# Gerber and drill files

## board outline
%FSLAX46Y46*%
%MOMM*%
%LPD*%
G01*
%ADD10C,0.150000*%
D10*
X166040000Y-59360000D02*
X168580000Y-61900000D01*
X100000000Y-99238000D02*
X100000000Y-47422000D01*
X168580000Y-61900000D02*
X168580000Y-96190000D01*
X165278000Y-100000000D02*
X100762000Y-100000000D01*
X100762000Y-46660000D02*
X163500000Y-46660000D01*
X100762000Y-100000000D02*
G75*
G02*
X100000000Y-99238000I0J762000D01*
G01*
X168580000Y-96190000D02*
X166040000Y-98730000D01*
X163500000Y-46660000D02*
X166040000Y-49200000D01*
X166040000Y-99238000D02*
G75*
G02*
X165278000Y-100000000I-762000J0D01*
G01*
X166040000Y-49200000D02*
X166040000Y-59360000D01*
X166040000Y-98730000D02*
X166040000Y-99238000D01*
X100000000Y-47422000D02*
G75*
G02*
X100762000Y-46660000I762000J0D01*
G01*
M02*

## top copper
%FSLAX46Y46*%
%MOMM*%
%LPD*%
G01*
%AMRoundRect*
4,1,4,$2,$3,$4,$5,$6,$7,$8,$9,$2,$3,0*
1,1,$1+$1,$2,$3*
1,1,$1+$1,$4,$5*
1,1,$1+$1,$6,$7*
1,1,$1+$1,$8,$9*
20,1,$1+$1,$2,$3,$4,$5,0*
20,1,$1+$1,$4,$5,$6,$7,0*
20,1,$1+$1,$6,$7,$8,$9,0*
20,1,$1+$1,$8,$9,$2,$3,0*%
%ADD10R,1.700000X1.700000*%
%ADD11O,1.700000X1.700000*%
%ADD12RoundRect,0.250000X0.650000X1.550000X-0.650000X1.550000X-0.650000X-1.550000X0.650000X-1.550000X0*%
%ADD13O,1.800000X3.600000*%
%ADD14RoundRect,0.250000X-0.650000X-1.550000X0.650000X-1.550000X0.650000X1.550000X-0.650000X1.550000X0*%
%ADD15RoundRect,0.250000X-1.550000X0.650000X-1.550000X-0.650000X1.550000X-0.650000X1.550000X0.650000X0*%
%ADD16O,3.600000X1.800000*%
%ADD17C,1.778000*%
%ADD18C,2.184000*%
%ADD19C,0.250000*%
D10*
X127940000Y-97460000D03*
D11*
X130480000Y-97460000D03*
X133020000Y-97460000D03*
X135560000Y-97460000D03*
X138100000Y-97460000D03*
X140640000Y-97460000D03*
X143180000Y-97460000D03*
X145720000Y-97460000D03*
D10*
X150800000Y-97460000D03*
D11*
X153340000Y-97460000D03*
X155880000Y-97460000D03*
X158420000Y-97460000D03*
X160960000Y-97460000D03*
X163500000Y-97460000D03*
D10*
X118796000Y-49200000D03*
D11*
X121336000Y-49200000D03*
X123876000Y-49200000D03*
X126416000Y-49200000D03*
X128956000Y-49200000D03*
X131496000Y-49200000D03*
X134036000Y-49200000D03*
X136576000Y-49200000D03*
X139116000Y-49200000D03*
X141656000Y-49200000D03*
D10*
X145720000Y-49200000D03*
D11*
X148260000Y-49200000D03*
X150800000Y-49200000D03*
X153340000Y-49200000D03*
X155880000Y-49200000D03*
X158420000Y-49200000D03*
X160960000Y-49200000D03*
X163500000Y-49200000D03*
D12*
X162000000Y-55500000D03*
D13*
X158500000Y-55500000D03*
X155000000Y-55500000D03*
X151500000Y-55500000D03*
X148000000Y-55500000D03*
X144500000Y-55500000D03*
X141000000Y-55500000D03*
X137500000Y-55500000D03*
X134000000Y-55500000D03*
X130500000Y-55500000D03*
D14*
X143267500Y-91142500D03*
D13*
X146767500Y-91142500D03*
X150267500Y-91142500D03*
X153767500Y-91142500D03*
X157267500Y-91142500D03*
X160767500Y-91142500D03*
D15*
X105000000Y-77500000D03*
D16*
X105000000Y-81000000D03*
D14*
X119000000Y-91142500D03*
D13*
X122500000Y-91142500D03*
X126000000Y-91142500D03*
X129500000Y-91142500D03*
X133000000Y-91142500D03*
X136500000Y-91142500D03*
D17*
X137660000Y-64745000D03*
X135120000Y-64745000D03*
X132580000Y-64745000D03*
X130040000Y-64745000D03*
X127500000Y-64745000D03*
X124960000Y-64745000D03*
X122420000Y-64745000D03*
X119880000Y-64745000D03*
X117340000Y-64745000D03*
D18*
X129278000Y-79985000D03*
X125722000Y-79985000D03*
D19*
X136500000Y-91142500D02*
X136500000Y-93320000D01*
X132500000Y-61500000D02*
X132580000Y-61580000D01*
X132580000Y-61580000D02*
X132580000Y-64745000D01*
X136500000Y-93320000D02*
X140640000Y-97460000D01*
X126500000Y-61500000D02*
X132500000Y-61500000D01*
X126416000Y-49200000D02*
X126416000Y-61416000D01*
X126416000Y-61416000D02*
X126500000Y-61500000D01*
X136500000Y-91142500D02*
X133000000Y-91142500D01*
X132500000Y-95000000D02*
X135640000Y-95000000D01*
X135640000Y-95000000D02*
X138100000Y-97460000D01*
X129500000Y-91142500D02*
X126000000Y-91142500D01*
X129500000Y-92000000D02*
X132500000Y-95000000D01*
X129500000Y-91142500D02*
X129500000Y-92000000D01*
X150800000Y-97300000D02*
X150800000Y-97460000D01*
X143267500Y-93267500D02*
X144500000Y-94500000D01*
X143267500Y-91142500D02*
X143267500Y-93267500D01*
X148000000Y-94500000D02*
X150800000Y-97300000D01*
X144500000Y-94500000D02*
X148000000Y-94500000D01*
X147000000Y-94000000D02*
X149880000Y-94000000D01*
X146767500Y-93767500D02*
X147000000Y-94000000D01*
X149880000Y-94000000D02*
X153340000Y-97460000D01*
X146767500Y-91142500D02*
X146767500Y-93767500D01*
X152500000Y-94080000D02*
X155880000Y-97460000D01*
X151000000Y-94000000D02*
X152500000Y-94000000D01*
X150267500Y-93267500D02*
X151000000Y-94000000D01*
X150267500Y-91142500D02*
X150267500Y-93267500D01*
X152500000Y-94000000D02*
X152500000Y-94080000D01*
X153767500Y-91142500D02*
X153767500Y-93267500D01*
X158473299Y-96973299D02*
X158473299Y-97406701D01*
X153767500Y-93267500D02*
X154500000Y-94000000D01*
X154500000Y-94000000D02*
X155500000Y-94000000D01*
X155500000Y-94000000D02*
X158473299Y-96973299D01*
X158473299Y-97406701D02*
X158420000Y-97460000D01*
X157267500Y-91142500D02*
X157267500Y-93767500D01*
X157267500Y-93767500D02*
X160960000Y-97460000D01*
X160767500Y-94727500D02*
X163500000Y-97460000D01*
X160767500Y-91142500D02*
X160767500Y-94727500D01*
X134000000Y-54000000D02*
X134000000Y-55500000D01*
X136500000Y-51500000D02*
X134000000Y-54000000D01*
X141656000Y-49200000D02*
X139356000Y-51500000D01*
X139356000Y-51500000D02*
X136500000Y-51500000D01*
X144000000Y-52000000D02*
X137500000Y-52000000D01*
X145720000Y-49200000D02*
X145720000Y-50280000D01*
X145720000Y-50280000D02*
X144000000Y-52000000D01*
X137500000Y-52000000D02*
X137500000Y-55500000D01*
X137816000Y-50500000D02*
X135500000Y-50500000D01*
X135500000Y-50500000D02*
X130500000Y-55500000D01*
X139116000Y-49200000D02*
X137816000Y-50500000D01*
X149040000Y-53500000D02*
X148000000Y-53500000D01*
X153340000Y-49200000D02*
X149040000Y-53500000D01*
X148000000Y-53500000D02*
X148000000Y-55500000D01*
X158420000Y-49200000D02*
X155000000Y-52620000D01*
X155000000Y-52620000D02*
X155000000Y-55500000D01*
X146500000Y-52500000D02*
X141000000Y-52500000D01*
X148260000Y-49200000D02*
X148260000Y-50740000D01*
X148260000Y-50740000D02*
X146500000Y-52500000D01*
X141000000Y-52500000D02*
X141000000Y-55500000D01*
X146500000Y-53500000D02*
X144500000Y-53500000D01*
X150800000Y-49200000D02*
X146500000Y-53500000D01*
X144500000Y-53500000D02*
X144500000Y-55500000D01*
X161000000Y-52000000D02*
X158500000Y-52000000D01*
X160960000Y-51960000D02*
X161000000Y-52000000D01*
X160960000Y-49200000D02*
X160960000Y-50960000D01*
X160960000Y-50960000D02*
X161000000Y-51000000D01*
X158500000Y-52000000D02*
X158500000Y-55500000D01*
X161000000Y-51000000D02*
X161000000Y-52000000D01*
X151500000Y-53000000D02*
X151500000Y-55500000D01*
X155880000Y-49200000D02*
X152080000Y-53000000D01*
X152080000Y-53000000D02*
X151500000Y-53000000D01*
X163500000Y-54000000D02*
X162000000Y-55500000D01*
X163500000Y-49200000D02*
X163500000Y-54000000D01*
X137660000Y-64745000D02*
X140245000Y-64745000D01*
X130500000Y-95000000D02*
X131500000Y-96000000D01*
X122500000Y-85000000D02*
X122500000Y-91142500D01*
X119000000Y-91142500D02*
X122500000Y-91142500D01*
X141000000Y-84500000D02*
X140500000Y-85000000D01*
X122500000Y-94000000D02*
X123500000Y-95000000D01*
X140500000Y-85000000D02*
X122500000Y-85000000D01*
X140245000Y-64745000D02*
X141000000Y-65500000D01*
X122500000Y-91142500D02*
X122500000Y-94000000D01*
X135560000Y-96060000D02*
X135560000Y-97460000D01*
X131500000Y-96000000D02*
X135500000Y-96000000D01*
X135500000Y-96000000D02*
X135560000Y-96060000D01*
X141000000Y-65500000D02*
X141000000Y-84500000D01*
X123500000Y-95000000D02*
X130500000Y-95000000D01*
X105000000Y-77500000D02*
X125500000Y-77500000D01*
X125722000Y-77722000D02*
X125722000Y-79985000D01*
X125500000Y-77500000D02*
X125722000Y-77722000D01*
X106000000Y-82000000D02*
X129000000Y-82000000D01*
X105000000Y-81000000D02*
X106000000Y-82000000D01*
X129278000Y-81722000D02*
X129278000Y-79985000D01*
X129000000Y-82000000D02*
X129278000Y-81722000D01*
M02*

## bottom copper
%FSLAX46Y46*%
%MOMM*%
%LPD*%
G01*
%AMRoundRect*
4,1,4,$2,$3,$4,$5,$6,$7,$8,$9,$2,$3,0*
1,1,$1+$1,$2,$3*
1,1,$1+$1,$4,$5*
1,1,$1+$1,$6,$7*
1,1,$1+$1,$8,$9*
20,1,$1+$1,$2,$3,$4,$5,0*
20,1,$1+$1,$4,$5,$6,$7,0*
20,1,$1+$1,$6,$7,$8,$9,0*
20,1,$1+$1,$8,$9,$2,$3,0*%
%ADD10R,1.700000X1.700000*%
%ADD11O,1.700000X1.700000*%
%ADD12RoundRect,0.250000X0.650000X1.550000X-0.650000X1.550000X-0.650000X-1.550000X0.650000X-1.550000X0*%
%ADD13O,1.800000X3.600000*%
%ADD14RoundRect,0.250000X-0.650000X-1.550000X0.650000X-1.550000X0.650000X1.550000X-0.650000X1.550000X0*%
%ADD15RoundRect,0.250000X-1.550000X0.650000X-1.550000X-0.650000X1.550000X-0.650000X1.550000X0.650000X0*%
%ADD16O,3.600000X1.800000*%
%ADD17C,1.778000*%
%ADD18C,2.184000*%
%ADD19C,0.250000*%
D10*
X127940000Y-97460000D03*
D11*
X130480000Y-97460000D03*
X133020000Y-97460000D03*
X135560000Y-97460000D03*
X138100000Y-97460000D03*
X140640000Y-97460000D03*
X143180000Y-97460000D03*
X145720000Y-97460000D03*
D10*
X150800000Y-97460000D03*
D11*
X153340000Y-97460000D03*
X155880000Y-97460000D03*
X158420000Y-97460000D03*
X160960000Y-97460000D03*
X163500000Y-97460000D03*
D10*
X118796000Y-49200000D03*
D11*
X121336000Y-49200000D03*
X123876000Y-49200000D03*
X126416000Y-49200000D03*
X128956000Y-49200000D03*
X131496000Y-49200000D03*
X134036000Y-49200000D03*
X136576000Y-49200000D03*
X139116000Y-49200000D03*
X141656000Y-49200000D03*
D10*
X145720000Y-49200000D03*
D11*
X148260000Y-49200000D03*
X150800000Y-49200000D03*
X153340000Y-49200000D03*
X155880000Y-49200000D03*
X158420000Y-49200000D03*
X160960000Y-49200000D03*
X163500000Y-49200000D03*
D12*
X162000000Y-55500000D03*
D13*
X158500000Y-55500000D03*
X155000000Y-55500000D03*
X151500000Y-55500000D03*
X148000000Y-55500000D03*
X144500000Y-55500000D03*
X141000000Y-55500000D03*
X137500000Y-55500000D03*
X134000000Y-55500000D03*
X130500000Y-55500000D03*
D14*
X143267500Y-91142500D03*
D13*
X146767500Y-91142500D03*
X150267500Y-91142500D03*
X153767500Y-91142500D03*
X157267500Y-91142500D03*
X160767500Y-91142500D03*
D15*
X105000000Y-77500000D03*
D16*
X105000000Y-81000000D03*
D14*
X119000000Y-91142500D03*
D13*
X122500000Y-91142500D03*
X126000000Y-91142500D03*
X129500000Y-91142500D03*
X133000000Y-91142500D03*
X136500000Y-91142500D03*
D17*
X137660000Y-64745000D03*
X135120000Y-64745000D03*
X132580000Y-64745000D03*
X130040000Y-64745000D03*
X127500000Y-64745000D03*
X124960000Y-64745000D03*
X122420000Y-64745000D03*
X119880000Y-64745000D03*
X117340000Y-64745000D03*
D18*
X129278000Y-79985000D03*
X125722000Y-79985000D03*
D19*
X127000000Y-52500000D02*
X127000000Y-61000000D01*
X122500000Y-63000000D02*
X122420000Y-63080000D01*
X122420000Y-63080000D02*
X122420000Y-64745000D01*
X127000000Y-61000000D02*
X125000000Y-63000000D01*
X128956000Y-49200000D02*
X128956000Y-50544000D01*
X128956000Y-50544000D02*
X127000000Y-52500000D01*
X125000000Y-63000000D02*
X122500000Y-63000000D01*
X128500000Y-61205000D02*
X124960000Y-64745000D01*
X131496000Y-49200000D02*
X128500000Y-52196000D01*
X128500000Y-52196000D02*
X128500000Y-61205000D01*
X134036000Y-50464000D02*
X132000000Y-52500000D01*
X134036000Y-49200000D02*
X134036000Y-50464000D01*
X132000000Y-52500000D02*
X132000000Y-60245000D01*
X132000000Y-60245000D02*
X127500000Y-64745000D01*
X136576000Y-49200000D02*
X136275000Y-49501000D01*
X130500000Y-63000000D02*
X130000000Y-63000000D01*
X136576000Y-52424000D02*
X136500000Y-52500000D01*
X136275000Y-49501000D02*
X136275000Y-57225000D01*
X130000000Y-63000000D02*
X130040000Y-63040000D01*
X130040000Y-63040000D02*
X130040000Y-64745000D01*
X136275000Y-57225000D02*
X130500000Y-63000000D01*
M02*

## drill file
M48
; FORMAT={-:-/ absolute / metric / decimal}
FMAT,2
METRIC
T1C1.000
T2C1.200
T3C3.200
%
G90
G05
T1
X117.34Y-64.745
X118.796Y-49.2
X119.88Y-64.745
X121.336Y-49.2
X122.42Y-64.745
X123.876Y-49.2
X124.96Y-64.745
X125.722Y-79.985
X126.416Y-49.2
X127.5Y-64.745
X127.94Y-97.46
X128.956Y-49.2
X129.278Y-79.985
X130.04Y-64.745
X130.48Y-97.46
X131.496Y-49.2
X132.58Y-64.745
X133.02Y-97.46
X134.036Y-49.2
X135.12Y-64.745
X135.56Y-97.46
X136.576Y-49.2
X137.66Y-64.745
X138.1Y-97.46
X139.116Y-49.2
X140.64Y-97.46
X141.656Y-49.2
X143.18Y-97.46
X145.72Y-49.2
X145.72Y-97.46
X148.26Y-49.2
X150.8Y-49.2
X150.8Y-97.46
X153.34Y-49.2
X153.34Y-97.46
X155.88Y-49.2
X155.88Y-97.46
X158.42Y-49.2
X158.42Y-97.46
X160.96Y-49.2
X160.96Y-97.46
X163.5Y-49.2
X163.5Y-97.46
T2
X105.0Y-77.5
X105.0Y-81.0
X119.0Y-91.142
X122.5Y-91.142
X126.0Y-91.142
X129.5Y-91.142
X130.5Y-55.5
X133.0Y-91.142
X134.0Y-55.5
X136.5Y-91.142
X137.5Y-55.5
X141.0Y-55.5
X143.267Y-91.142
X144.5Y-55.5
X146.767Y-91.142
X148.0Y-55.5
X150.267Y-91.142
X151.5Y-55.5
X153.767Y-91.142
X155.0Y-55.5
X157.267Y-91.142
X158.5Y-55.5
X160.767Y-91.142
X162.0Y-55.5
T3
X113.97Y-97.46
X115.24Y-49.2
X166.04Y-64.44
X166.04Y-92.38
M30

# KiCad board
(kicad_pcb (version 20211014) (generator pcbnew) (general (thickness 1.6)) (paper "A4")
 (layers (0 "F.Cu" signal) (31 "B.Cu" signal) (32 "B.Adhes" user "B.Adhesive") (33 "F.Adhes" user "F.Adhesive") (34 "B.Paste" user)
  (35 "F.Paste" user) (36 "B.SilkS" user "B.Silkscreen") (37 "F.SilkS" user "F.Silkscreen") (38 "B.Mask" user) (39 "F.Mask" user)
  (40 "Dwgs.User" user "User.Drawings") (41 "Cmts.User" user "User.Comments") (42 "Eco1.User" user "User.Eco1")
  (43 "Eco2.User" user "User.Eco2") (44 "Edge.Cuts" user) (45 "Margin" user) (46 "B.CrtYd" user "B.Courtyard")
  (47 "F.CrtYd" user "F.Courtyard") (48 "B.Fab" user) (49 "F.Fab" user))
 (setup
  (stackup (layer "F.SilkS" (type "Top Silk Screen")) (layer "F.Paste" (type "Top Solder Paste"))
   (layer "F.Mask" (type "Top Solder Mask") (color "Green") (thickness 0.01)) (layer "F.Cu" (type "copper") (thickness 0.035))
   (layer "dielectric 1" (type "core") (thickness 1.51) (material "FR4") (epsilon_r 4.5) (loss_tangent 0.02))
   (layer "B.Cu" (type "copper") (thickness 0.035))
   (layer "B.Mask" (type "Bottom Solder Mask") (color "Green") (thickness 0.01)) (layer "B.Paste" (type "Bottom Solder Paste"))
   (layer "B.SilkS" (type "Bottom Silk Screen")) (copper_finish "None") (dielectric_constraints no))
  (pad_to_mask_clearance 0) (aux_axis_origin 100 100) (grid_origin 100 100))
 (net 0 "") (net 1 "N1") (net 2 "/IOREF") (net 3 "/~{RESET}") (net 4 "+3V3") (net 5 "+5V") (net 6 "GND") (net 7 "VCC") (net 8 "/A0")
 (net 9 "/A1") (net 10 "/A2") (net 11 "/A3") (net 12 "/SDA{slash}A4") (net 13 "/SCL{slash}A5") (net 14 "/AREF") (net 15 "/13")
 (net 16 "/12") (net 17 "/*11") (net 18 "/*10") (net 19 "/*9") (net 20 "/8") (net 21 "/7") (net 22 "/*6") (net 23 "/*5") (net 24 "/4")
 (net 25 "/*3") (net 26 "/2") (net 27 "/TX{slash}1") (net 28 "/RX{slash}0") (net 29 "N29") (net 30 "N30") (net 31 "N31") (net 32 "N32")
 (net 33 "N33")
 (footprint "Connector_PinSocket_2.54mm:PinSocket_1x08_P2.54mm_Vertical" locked (layer "F.Cu") (at 127.94 97.46 90)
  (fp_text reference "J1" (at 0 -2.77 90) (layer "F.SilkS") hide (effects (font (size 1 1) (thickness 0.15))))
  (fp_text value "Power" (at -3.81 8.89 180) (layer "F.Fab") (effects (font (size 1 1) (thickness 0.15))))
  (pad "1" thru_hole rect locked (at 0 0 90) (size 1.7 1.7) (drill 1) (layers *.Cu *.Mask) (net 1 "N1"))
  (pad "2" thru_hole oval locked (at 0 2.54 90) (size 1.7 1.7) (drill 1) (layers *.Cu *.Mask) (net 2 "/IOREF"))
  (pad "3" thru_hole oval locked (at 0 5.08 90) (size 1.7 1.7) (drill 1) (layers *.Cu *.Mask) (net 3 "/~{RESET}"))
  (pad "4" thru_hole oval locked (at 0 7.62 90) (size 1.7 1.7) (drill 1) (layers *.Cu *.Mask) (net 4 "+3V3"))
  (pad "5" thru_hole oval locked (at 0 10.16 90) (size 1.7 1.7) (drill 1) (layers *.Cu *.Mask) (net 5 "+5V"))
  (pad "6" thru_hole oval locked (at 0 12.7 90) (size 1.7 1.7) (drill 1) (layers *.Cu *.Mask) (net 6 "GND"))
  (pad "7" thru_hole oval locked (at 0 15.24 90) (size 1.7 1.7) (drill 1) (layers *.Cu *.Mask) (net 6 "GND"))
  (pad "8" thru_hole oval locked (at 0 17.78 90) (size 1.7 1.7) (drill 1) (layers *.Cu *.Mask) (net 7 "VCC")))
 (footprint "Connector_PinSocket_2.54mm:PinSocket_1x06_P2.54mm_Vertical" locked (layer "F.Cu") (at 150.8 97.46 90)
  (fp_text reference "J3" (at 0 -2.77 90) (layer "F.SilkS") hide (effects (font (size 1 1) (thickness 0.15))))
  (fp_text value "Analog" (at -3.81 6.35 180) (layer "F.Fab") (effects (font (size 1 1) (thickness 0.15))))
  (pad "1" thru_hole rect locked (at 0 0 90) (size 1.7 1.7) (drill 1) (layers *.Cu *.Mask) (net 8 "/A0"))
  (pad "2" thru_hole oval locked (at 0 2.54 90) (size 1.7 1.7) (drill 1) (layers *.Cu *.Mask) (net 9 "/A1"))
  (pad "3" thru_hole oval locked (at 0 5.08 90) (size 1.7 1.7) (drill 1) (layers *.Cu *.Mask) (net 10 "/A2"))
  (pad "4" thru_hole oval locked (at 0 7.62 90) (size 1.7 1.7) (drill 1) (layers *.Cu *.Mask) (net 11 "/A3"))
  (pad "5" thru_hole oval locked (at 0 10.16 90) (size 1.7 1.7) (drill 1) (layers *.Cu *.Mask) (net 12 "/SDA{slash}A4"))
  (pad "6" thru_hole oval locked (at 0 12.7 90) (size 1.7 1.7) (drill 1) (layers *.Cu *.Mask) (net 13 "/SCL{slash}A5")))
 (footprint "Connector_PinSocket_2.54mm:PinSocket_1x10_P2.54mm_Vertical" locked (layer "F.Cu") (at 118.796 49.2 90)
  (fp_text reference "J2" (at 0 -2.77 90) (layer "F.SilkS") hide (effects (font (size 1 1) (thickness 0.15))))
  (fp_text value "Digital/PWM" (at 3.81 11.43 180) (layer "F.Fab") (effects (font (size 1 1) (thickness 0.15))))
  (pad "1" thru_hole rect locked (at 0 0 90) (size 1.7 1.7) (drill 1) (layers *.Cu *.Mask) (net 13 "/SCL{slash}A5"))
  (pad "2" thru_hole oval locked (at 0 2.54 90) (size 1.7 1.7) (drill 1) (layers *.Cu *.Mask) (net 12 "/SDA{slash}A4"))
  (pad "3" thru_hole oval locked (at 0 5.08 90) (size 1.7 1.7) (drill 1) (layers *.Cu *.Mask) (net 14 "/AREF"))
  (pad "4" thru_hole oval locked (at 0 7.62 90) (size 1.7 1.7) (drill 1) (layers *.Cu *.Mask) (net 6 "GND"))
  (pad "5" thru_hole oval locked (at 0 10.16 90) (size 1.7 1.7) (drill 1) (layers *.Cu *.Mask) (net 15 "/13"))
  (pad "6" thru_hole oval locked (at 0 12.7 90) (size 1.7 1.7) (drill 1) (layers *.Cu *.Mask) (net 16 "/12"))
  (pad "7" thru_hole oval locked (at 0 15.24 90) (size 1.7 1.7) (drill 1) (layers *.Cu *.Mask) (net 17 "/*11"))
  (pad "8" thru_hole oval locked (at 0 17.78 90) (size 1.7 1.7) (drill 1) (layers *.Cu *.Mask) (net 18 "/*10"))
  (pad "9" thru_hole oval locked (at 0 20.32 90) (size 1.7 1.7) (drill 1) (layers *.Cu *.Mask) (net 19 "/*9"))
  (pad "10" thru_hole oval locked (at 0 22.86 90) (size 1.7 1.7) (drill 1) (layers *.Cu *.Mask) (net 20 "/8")))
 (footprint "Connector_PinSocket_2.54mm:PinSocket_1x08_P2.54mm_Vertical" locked (layer "F.Cu") (at 145.72 49.2 90)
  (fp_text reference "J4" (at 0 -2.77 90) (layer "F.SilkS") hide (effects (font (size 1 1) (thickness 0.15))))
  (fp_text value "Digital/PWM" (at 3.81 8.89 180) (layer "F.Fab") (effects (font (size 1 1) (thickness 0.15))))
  (pad "1" thru_hole rect locked (at 0 0 90) (size 1.7 1.7) (drill 1) (layers *.Cu *.Mask) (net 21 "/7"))
  (pad "2" thru_hole oval locked (at 0 2.54 90) (size 1.7 1.7) (drill 1) (layers *.Cu *.Mask) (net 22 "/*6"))
  (pad "3" thru_hole oval locked (at 0 5.08 90) (size 1.7 1.7) (drill 1) (layers *.Cu *.Mask) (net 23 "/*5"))
  (pad "4" thru_hole oval locked (at 0 7.62 90) (size 1.7 1.7) (drill 1) (layers *.Cu *.Mask) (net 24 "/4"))
  (pad "5" thru_hole oval locked (at 0 10.16 90) (size 1.7 1.7) (drill 1) (layers *.Cu *.Mask) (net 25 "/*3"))
  (pad "6" thru_hole oval locked (at 0 12.7 90) (size 1.7 1.7) (drill 1) (layers *.Cu *.Mask) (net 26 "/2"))
  (pad "7" thru_hole oval locked (at 0 15.24 90) (size 1.7 1.7) (drill 1) (layers *.Cu *.Mask) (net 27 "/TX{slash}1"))
  (pad "8" thru_hole oval locked (at 0 17.78 90) (size 1.7 1.7) (drill 1) (layers *.Cu *.Mask) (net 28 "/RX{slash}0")))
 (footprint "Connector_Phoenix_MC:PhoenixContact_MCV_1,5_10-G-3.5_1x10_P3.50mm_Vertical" (layer "F.Cu") (at 162 55.5 180)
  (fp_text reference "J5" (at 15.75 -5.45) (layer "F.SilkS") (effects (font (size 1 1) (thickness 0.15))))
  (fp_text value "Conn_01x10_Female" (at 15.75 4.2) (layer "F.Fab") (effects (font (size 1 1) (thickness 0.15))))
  (pad "1" thru_hole roundrect (at 0 0 180) (size 1.8 3.6) (drill 1.2) (layers *.Cu *.Mask) (roundrect_rratio 0.138889)
   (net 28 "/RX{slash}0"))
  (pad "2" thru_hole oval (at 3.5 0 180) (size 1.8 3.6) (drill 1.2) (layers *.Cu *.Mask) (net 27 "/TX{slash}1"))
  (pad "3" thru_hole oval (at 7 0 180) (size 1.8 3.6) (drill 1.2) (layers *.Cu *.Mask) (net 26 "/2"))
  (pad "4" thru_hole oval (at 10.5 0 180) (size 1.8 3.6) (drill 1.2) (layers *.Cu *.Mask) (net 25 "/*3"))
  (pad "5" thru_hole oval (at 14 0 180) (size 1.8 3.6) (drill 1.2) (layers *.Cu *.Mask) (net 24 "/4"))
  (pad "6" thru_hole oval (at 17.5 0 180) (size 1.8 3.6) (drill 1.2) (layers *.Cu *.Mask) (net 23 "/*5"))
  (pad "7" thru_hole oval (at 21 0 180) (size 1.8 3.6) (drill 1.2) (layers *.Cu *.Mask) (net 22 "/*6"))
  (pad "8" thru_hole oval (at 24.5 0 180) (size 1.8 3.6) (drill 1.2) (layers *.Cu *.Mask) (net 21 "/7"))
  (pad "9" thru_hole oval (at 28 0 180) (size 1.8 3.6) (drill 1.2) (layers *.Cu *.Mask) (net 20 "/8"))
  (pad "10" thru_hole oval (at 31.5 0 180) (size 1.8 3.6) (drill 1.2) (layers *.Cu *.Mask) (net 19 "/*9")))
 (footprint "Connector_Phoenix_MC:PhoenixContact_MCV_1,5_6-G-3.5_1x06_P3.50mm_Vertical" (layer "F.Cu") (at 143.2675 91.1425)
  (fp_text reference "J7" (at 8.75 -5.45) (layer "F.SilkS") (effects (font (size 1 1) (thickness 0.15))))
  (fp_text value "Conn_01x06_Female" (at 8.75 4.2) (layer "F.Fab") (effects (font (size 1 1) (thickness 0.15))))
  (pad "1" thru_hole roundrect (at 0 0) (size 1.8 3.6) (drill 1.2) (layers *.Cu *.Mask) (roundrect_rratio 0.138889) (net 8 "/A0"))
  (pad "2" thru_hole oval (at 3.5 0) (size 1.8 3.6) (drill 1.2) (layers *.Cu *.Mask) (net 9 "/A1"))
  (pad "3" thru_hole oval (at 7 0) (size 1.8 3.6) (drill 1.2) (layers *.Cu *.Mask) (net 10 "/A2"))
  (pad "4" thru_hole oval (at 10.5 0) (size 1.8 3.6) (drill 1.2) (layers *.Cu *.Mask) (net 11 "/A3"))
  (pad "5" thru_hole oval (at 14 0) (size 1.8 3.6) (drill 1.2) (layers *.Cu *.Mask) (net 12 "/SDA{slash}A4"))
  (pad "6" thru_hole oval (at 17.5 0) (size 1.8 3.6) (drill 1.2) (layers *.Cu *.Mask) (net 13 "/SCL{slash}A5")))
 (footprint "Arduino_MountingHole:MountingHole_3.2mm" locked (layer "F.Cu") (at 115.24 49.2)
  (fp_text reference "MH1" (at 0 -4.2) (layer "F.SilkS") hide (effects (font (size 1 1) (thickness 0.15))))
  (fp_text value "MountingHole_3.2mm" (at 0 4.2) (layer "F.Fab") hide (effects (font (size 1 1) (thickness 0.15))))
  (pad "" np_thru_hole circle locked (at 0 0) (size 3.2 3.2) (drill 3.2) (layers *.Cu *.Mask)))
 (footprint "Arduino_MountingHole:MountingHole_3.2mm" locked (layer "F.Cu") (at 113.97 97.46)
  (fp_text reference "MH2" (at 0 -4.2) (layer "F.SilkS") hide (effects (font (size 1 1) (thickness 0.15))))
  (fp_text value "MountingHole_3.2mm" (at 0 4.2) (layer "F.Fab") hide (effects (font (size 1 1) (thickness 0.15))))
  (pad "" np_thru_hole circle locked (at 0 0) (size 3.2 3.2) (drill 3.2) (layers *.Cu *.Mask)))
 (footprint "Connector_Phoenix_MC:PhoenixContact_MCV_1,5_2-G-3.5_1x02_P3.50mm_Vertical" (layer "F.Cu") (at 105 77.5 -90)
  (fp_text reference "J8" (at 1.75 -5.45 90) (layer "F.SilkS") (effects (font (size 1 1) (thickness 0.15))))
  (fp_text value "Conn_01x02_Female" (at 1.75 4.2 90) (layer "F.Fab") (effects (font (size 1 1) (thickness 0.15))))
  (pad "1" thru_hole roundrect (at 0 0 270) (size 1.8 3.6) (drill 1.2) (layers *.Cu *.Mask) (roundrect_rratio 0.138889) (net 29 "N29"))
  (pad "2" thru_hole oval (at 3.5 0 270) (size 1.8 3.6) (drill 1.2) (layers *.Cu *.Mask) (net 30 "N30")))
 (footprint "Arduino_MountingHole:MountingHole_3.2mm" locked (layer "F.Cu") (at 166.04 64.44)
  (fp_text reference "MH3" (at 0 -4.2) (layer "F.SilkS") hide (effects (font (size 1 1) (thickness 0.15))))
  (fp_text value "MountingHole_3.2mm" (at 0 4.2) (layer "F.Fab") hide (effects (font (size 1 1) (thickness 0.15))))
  (pad "" np_thru_hole circle locked (at 0 0) (size 3.2 3.2) (drill 3.2) (layers *.Cu *.Mask)))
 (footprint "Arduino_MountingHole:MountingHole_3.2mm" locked (layer "F.Cu") (at 166.04 92.38)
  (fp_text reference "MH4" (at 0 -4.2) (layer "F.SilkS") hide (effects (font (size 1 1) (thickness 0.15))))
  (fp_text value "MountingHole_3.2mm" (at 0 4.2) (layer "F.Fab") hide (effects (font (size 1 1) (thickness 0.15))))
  (pad "" np_thru_hole circle locked (at 0 0) (size 3.2 3.2) (drill 3.2) (layers *.Cu *.Mask)))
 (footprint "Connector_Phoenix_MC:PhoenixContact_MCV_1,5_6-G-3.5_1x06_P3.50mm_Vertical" (layer "F.Cu") (at 119 91.1425)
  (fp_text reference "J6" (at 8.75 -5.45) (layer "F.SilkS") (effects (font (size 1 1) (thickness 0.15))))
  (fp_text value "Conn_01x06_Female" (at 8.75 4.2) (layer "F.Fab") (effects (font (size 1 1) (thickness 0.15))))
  (pad "1" thru_hole roundrect (at 0 0) (size 1.8 3.6) (drill 1.2) (layers *.Cu *.Mask) (roundrect_rratio 0.138889) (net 4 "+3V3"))
  (pad "2" thru_hole oval (at 3.5 0) (size 1.8 3.6) (drill 1.2) (layers *.Cu *.Mask) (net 4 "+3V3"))
  (pad "3" thru_hole oval (at 7 0) (size 1.8 3.6) (drill 1.2) (layers *.Cu *.Mask) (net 5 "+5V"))
  (pad "4" thru_hole oval (at 10.5 0) (size 1.8 3.6) (drill 1.2) (layers *.Cu *.Mask) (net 5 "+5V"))
  (pad "5" thru_hole oval (at 14 0) (size 1.8 3.6) (drill 1.2) (layers *.Cu *.Mask) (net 6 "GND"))
  (pad "6" thru_hole oval (at 17.5 0) (size 1.8 3.6) (drill 1.2) (layers *.Cu *.Mask) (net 6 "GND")))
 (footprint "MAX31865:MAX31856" (layer "F.Cu") (at 127.5 73 180)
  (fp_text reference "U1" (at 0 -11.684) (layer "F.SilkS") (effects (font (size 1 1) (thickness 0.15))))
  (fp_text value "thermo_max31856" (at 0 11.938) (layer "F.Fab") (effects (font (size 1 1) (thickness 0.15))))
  (pad "1" thru_hole circle (at -10.16 8.255 180) (size 1.778 1.778) (drill 1) (layers *.Cu *.Mask) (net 4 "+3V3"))
  (pad "2" thru_hole circle (at -7.62 8.255 180) (size 1.778 1.778) (drill 1) (layers *.Cu *.Mask) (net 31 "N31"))
  (pad "3" thru_hole circle (at -5.08 8.255 180) (size 1.778 1.778) (drill 1) (layers *.Cu *.Mask) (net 6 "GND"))
  (pad "4" thru_hole circle (at -2.54 8.255 180) (size 1.778 1.778) (drill 1) (layers *.Cu *.Mask) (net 18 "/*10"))
  (pad "5" thru_hole circle (at 0 8.255 180) (size 1.778 1.778) (drill 1) (layers *.Cu *.Mask) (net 17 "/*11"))
  (pad "6" thru_hole circle (at 2.54 8.255 180) (size 1.778 1.778) (drill 1) (layers *.Cu *.Mask) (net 16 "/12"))
  (pad "7" thru_hole circle (at 5.08 8.255 180) (size 1.778 1.778) (drill 1) (layers *.Cu *.Mask) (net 15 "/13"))
  (pad "8" thru_hole circle (at 7.62 8.255 180) (size 1.778 1.778) (drill 1) (layers *.Cu *.Mask) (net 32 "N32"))
  (pad "9" thru_hole circle (at 10.16 8.255 180) (size 1.778 1.778) (drill 1) (layers *.Cu *.Mask) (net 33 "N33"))
  (pad "10" thru_hole circle (at -1.778 -6.985 180) (size 2.184 2.184) (drill 1) (layers *.Cu *.Mask) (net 30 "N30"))
  (pad "11" thru_hole circle (at 1.778 -6.985 180) (size 2.184 2.184) (drill 1) (layers *.Cu *.Mask) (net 29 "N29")))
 (gr_line (start 166.04 59.36) (end 168.58 61.9) (layer "Edge.Cuts") (width 0.15))
 (gr_line (start 100 99.238) (end 100 47.422) (layer "Edge.Cuts") (width 0.15))
 (gr_line (start 168.58 61.9) (end 168.58 96.19) (layer "Edge.Cuts") (width 0.15))
 (gr_line (start 165.278 100) (end 100.762 100) (layer "Edge.Cuts") (width 0.15))
 (gr_line (start 100.762 46.66) (end 163.5 46.66) (layer "Edge.Cuts") (width 0.15))
 (gr_arc (start 100.762 100) (mid 100.223185 99.776815) (end 100 99.238) (layer "Edge.Cuts") (width 0.15))
 (gr_line (start 168.58 96.19) (end 166.04 98.73) (layer "Edge.Cuts") (width 0.15))
 (gr_line (start 163.5 46.66) (end 166.04 49.2) (layer "Edge.Cuts") (width 0.15))
 (gr_arc (start 166.04 99.238) (mid 165.816815 99.776815) (end 165.278 100) (layer "Edge.Cuts") (width 0.15))
 (gr_line (start 166.04 49.2) (end 166.04 59.36) (layer "Edge.Cuts") (width 0.15))
 (gr_line (start 166.04 98.73) (end 166.04 99.238) (layer "Edge.Cuts") (width 0.15))
 (gr_arc (start 100 47.422) (mid 100.223185 46.883185) (end 100.762 46.66) (layer "Edge.Cuts") (width 0.15))
 (segment (start 136.5 91.1425) (end 136.5 93.32) (width 0.25) (layer "F.Cu") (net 6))
 (segment (start 132.5 61.5) (end 132.58 61.58) (width 0.25) (layer "F.Cu") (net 6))
 (segment (start 132.58 61.58) (end 132.58 64.745) (width 0.25) (layer "F.Cu") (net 6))
 (segment (start 136.5 93.32) (end 140.64 97.46) (width 0.25) (layer "F.Cu") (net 6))
 (segment (start 126.5 61.5) (end 132.5 61.5) (width 0.25) (layer "F.Cu") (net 6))
 (segment (start 126.416 49.2) (end 126.416 61.416) (width 0.25) (layer "F.Cu") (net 6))
 (segment (start 126.416 61.416) (end 126.5 61.5) (width 0.25) (layer "F.Cu") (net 6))
 (segment (start 136.5 91.1425) (end 133 91.1425) (width 0.25) (layer "F.Cu") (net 6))
 (segment (start 132.5 95) (end 135.64 95) (width 0.25) (layer "F.Cu") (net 5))
 (segment (start 135.64 95) (end 138.1 97.46) (width 0.25) (layer "F.Cu") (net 5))
 (segment (start 129.5 91.1425) (end 126 91.1425) (width 0.25) (layer "F.Cu") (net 5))
 (segment (start 129.5 92) (end 132.5 95) (width 0.25) (layer "F.Cu") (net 5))
 (segment (start 129.5 91.1425) (end 129.5 92) (width 0.25) (layer "F.Cu") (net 5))
 (segment (start 150.8 97.3) (end 150.8 97.46) (width 0.25) (layer "F.Cu") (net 8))
 (segment (start 143.2675 93.2675) (end 144.5 94.5) (width 0.25) (layer "F.Cu") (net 8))
 (segment (start 143.2675 91.1425) (end 143.2675 93.2675) (width 0.25) (layer "F.Cu") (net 8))
 (segment (start 148 94.5) (end 150.8 97.3) (width 0.25) (layer "F.Cu") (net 8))
 (segment (start 144.5 94.5) (end 148 94.5) (width 0.25) (layer "F.Cu") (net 8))
 (segment (start 147 94) (end 149.88 94) (width 0.25) (layer "F.Cu") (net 9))
 (segment (start 146.7675 93.7675) (end 147 94) (width 0.25) (layer "F.Cu") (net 9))
 (segment (start 149.88 94) (end 153.34 97.46) (width 0.25) (layer "F.Cu") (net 9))
 (segment (start 146.7675 91.1425) (end 146.7675 93.7675) (width 0.25) (layer "F.Cu") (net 9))
 (segment (start 152.5 94.08) (end 155.88 97.46) (width 0.25) (layer "F.Cu") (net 10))
 (segment (start 151 94) (end 152.5 94) (width 0.25) (layer "F.Cu") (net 10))
 (segment (start 150.2675 93.2675) (end 151 94) (width 0.25) (layer "F.Cu") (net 10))
 (segment (start 150.2675 91.1425) (end 150.2675 93.2675) (width 0.25) (layer "F.Cu") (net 10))
 (segment (start 152.5 94) (end 152.5 94.08) (width 0.25) (layer "F.Cu") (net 10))
 (segment (start 153.7675 91.1425) (end 153.7675 93.2675) (width 0.25) (layer "F.Cu") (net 11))
 (segment (start 158.473299 96.973299) (end 158.473299 97.406701) (width 0.25) (layer "F.Cu") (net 11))
 (segment (start 153.7675 93.2675) (end 154.5 94) (width 0.25) (layer "F.Cu") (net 11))
 (segment (start 154.5 94) (end 155.5 94) (width 0.25) (layer "F.Cu") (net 11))
 (segment (start 155.5 94) (end 158.473299 96.973299) (width 0.25) (layer "F.Cu") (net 11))
 (segment (start 158.473299 97.406701) (end 158.42 97.46) (width 0.25) (layer "F.Cu") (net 11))
 (segment (start 157.2675 91.1425) (end 157.2675 93.7675) (width 0.25) (layer "F.Cu") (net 12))
 (segment (start 157.2675 93.7675) (end 160.96 97.46) (width 0.25) (layer "F.Cu") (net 12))
 (segment (start 160.7675 94.7275) (end 163.5 97.46) (width 0.25) (layer "F.Cu") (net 13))
 (segment (start 160.7675 91.1425) (end 160.7675 94.7275) (width 0.25) (layer "F.Cu") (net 13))
 (segment (start 127 52.5) (end 127 61) (width 0.25) (layer "B.Cu") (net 15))
 (segment (start 122.5 63) (end 122.42 63.08) (width 0.25) (layer "B.Cu") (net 15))
 (segment (start 122.42 63.08) (end 122.42 64.745) (width 0.25) (layer "B.Cu") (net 15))
 (segment (start 127 61) (end 125 63) (width 0.25) (layer "B.Cu") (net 15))
 (segment (start 128.956 49.2) (end 128.956 50.544) (width 0.25) (layer "B.Cu") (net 15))
 (segment (start 128.956 50.544) (end 127 52.5) (width 0.25) (layer "B.Cu") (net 15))
 (segment (start 125 63) (end 122.5 63) (width 0.25) (layer "B.Cu") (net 15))
 (segment (start 128.5 61.205) (end 124.96 64.745) (width 0.25) (layer "B.Cu") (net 16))
 (segment (start 131.496 49.2) (end 128.5 52.196) (width 0.25) (layer "B.Cu") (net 16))
 (segment (start 128.5 52.196) (end 128.5 61.205) (width 0.25) (layer "B.Cu") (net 16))
 (segment (start 134 54) (end 134 55.5) (width 0.25) (layer "F.Cu") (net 20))
 (segment (start 136.5 51.5) (end 134 54) (width 0.25) (layer "F.Cu") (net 20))
 (segment (start 141.656 49.2) (end 139.356 51.5) (width 0.25) (layer "F.Cu") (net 20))
 (segment (start 139.356 51.5) (end 136.5 51.5) (width 0.25) (layer "F.Cu") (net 20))
 (segment (start 144 52) (end 137.5 52) (width 0.25) (layer "F.Cu") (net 21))
 (segment (start 145.72 49.2) (end 145.72 50.28) (width 0.25) (layer "F.Cu") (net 21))
 (segment (start 145.72 50.28) (end 144 52) (width 0.25) (layer "F.Cu") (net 21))
 (segment (start 137.5 52) (end 137.5 55.5) (width 0.25) (layer "F.Cu") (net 21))
 (segment (start 134.036 50.464) (end 132 52.5) (width 0.25) (layer "B.Cu") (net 17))
 (segment (start 134.036 49.2) (end 134.036 50.464) (width 0.25) (layer "B.Cu") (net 17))
 (segment (start 132 52.5) (end 132 60.245) (width 0.25) (layer "B.Cu") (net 17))
 (segment (start 132 60.245) (end 127.5 64.745) (width 0.25) (layer "B.Cu") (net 17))
 (segment (start 136.576 49.2) (end 136.275 49.501) (width 0.25) (layer "B.Cu") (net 18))
 (segment (start 130.5 63) (end 130 63) (width 0.25) (layer "B.Cu") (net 18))
 (segment (start 136.576 52.424) (end 136.5 52.5) (width 0.25) (layer "B.Cu") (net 18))
 (segment (start 136.275 49.501) (end 136.275 57.225) (width 0.25) (layer "B.Cu") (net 18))
 (segment (start 130 63) (end 130.04 63.04) (width 0.25) (layer "B.Cu") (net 18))
 (segment (start 130.04 63.04) (end 130.04 64.745) (width 0.25) (layer "B.Cu") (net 18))
 (segment (start 136.275 57.225) (end 130.5 63) (width 0.25) (layer "B.Cu") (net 18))
 (segment (start 137.816 50.5) (end 135.5 50.5) (width 0.25) (layer "F.Cu") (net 19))
 (segment (start 135.5 50.5) (end 130.5 55.5) (width 0.25) (layer "F.Cu") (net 19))
 (segment (start 139.116 49.2) (end 137.816 50.5) (width 0.25) (layer "F.Cu") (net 19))
 (segment (start 149.04 53.5) (end 148 53.5) (width 0.25) (layer "F.Cu") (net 24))
 (segment (start 153.34 49.2) (end 149.04 53.5) (width 0.25) (layer "F.Cu") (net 24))
 (segment (start 148 53.5) (end 148 55.5) (width 0.25) (layer "F.Cu") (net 24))
 (segment (start 158.42 49.2) (end 155 52.62) (width 0.25) (layer "F.Cu") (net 26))
 (segment (start 155 52.62) (end 155 55.5) (width 0.25) (layer "F.Cu") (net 26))
 (segment (start 146.5 52.5) (end 141 52.5) (width 0.25) (layer "F.Cu") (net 22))
 (segment (start 148.26 49.2) (end 148.26 50.74) (width 0.25) (layer "F.Cu") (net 22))
 (segment (start 148.26 50.74) (end 146.5 52.5) (width 0.25) (layer "F.Cu") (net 22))
 (segment (start 141 52.5) (end 141 55.5) (width 0.25) (layer "F.Cu") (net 22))
 (segment (start 146.5 53.5) (end 144.5 53.5) (width 0.25) (layer "F.Cu") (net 23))
 (segment (start 150.8 49.2) (end 146.5 53.5) (width 0.25) (layer "F.Cu") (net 23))
 (segment (start 144.5 53.5) (end 144.5 55.5) (width 0.25) (layer "F.Cu") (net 23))
 (segment (start 161 52) (end 158.5 52) (width 0.25) (layer "F.Cu") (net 27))
 (segment (start 160.96 51.96) (end 161 52) (width 0.25) (layer "F.Cu") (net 27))
 (segment (start 160.96 49.2) (end 160.96 50.96) (width 0.25) (layer "F.Cu") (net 27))
 (segment (start 160.96 50.96) (end 161 51) (width 0.25) (layer "F.Cu") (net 27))
 (segment (start 158.5 52) (end 158.5 55.5) (width 0.25) (layer "F.Cu") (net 27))
 (segment (start 161 51) (end 161 52) (width 0.25) (layer "F.Cu") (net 27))
 (segment (start 151.5 53) (end 151.5 55.5) (width 0.25) (layer "F.Cu") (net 25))
 (segment (start 155.88 49.2) (end 152.08 53) (width 0.25) (layer "F.Cu") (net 25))
 (segment (start 152.08 53) (end 151.5 53) (width 0.25) (layer "F.Cu") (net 25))
 (segment (start 163.5 54) (end 162 55.5) (width 0.25) (layer "F.Cu") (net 28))
 (segment (start 163.5 49.2) (end 163.5 54) (width 0.25) (layer "F.Cu") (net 28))
 (segment (start 137.66 64.745) (end 140.245 64.745) (width 0.25) (layer "F.Cu") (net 4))
 (segment (start 130.5 95) (end 131.5 96) (width 0.25) (layer "F.Cu") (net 4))
 (segment (start 122.5 85) (end 122.5 91.1425) (width 0.25) (layer "F.Cu") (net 4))
 (segment (start 119 91.1425) (end 122.5 91.1425) (width 0.25) (layer "F.Cu") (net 4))
 (segment (start 141 84.5) (end 140.5 85) (width 0.25) (layer "F.Cu") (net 4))
 (segment (start 122.5 94) (end 123.5 95) (width 0.25) (layer "F.Cu") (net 4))
 (segment (start 140.5 85) (end 122.5 85) (width 0.25) (layer "F.Cu") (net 4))
 (segment (start 140.245 64.745) (end 141 65.5) (width 0.25) (layer "F.Cu") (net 4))
 (segment (start 122.5 91.1425) (end 122.5 94) (width 0.25) (layer "F.Cu") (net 4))
 (segment (start 135.56 96.06) (end 135.56 97.46) (width 0.25) (layer "F.Cu") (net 4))
 (segment (start 131.5 96) (end 135.5 96) (width 0.25) (layer "F.Cu") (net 4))
 (segment (start 135.5 96) (end 135.56 96.06) (width 0.25) (layer "F.Cu") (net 4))
 (segment (start 141 65.5) (end 141 84.5) (width 0.25) (layer "F.Cu") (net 4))
 (segment (start 123.5 95) (end 130.5 95) (width 0.25) (layer "F.Cu") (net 4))
 (segment (start 105 77.5) (end 125.5 77.5) (width 0.25) (layer "F.Cu") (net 29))
 (segment (start 125.722 77.722) (end 125.722 79.985) (width 0.25) (layer "F.Cu") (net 29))
 (segment (start 125.5 77.5) (end 125.722 77.722) (width 0.25) (layer "F.Cu") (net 29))
 (segment (start 106 82) (end 129 82) (width 0.25) (layer "F.Cu") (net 30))
 (segment (start 105 81) (end 106 82) (width 0.25) (layer "F.Cu") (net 30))
 (segment (start 129.278 81.722) (end 129.278 79.985) (width 0.25) (layer "F.Cu") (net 30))
 (segment (start 129 82) (end 129.278 81.722) (width 0.25) (layer "F.Cu") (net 30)))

